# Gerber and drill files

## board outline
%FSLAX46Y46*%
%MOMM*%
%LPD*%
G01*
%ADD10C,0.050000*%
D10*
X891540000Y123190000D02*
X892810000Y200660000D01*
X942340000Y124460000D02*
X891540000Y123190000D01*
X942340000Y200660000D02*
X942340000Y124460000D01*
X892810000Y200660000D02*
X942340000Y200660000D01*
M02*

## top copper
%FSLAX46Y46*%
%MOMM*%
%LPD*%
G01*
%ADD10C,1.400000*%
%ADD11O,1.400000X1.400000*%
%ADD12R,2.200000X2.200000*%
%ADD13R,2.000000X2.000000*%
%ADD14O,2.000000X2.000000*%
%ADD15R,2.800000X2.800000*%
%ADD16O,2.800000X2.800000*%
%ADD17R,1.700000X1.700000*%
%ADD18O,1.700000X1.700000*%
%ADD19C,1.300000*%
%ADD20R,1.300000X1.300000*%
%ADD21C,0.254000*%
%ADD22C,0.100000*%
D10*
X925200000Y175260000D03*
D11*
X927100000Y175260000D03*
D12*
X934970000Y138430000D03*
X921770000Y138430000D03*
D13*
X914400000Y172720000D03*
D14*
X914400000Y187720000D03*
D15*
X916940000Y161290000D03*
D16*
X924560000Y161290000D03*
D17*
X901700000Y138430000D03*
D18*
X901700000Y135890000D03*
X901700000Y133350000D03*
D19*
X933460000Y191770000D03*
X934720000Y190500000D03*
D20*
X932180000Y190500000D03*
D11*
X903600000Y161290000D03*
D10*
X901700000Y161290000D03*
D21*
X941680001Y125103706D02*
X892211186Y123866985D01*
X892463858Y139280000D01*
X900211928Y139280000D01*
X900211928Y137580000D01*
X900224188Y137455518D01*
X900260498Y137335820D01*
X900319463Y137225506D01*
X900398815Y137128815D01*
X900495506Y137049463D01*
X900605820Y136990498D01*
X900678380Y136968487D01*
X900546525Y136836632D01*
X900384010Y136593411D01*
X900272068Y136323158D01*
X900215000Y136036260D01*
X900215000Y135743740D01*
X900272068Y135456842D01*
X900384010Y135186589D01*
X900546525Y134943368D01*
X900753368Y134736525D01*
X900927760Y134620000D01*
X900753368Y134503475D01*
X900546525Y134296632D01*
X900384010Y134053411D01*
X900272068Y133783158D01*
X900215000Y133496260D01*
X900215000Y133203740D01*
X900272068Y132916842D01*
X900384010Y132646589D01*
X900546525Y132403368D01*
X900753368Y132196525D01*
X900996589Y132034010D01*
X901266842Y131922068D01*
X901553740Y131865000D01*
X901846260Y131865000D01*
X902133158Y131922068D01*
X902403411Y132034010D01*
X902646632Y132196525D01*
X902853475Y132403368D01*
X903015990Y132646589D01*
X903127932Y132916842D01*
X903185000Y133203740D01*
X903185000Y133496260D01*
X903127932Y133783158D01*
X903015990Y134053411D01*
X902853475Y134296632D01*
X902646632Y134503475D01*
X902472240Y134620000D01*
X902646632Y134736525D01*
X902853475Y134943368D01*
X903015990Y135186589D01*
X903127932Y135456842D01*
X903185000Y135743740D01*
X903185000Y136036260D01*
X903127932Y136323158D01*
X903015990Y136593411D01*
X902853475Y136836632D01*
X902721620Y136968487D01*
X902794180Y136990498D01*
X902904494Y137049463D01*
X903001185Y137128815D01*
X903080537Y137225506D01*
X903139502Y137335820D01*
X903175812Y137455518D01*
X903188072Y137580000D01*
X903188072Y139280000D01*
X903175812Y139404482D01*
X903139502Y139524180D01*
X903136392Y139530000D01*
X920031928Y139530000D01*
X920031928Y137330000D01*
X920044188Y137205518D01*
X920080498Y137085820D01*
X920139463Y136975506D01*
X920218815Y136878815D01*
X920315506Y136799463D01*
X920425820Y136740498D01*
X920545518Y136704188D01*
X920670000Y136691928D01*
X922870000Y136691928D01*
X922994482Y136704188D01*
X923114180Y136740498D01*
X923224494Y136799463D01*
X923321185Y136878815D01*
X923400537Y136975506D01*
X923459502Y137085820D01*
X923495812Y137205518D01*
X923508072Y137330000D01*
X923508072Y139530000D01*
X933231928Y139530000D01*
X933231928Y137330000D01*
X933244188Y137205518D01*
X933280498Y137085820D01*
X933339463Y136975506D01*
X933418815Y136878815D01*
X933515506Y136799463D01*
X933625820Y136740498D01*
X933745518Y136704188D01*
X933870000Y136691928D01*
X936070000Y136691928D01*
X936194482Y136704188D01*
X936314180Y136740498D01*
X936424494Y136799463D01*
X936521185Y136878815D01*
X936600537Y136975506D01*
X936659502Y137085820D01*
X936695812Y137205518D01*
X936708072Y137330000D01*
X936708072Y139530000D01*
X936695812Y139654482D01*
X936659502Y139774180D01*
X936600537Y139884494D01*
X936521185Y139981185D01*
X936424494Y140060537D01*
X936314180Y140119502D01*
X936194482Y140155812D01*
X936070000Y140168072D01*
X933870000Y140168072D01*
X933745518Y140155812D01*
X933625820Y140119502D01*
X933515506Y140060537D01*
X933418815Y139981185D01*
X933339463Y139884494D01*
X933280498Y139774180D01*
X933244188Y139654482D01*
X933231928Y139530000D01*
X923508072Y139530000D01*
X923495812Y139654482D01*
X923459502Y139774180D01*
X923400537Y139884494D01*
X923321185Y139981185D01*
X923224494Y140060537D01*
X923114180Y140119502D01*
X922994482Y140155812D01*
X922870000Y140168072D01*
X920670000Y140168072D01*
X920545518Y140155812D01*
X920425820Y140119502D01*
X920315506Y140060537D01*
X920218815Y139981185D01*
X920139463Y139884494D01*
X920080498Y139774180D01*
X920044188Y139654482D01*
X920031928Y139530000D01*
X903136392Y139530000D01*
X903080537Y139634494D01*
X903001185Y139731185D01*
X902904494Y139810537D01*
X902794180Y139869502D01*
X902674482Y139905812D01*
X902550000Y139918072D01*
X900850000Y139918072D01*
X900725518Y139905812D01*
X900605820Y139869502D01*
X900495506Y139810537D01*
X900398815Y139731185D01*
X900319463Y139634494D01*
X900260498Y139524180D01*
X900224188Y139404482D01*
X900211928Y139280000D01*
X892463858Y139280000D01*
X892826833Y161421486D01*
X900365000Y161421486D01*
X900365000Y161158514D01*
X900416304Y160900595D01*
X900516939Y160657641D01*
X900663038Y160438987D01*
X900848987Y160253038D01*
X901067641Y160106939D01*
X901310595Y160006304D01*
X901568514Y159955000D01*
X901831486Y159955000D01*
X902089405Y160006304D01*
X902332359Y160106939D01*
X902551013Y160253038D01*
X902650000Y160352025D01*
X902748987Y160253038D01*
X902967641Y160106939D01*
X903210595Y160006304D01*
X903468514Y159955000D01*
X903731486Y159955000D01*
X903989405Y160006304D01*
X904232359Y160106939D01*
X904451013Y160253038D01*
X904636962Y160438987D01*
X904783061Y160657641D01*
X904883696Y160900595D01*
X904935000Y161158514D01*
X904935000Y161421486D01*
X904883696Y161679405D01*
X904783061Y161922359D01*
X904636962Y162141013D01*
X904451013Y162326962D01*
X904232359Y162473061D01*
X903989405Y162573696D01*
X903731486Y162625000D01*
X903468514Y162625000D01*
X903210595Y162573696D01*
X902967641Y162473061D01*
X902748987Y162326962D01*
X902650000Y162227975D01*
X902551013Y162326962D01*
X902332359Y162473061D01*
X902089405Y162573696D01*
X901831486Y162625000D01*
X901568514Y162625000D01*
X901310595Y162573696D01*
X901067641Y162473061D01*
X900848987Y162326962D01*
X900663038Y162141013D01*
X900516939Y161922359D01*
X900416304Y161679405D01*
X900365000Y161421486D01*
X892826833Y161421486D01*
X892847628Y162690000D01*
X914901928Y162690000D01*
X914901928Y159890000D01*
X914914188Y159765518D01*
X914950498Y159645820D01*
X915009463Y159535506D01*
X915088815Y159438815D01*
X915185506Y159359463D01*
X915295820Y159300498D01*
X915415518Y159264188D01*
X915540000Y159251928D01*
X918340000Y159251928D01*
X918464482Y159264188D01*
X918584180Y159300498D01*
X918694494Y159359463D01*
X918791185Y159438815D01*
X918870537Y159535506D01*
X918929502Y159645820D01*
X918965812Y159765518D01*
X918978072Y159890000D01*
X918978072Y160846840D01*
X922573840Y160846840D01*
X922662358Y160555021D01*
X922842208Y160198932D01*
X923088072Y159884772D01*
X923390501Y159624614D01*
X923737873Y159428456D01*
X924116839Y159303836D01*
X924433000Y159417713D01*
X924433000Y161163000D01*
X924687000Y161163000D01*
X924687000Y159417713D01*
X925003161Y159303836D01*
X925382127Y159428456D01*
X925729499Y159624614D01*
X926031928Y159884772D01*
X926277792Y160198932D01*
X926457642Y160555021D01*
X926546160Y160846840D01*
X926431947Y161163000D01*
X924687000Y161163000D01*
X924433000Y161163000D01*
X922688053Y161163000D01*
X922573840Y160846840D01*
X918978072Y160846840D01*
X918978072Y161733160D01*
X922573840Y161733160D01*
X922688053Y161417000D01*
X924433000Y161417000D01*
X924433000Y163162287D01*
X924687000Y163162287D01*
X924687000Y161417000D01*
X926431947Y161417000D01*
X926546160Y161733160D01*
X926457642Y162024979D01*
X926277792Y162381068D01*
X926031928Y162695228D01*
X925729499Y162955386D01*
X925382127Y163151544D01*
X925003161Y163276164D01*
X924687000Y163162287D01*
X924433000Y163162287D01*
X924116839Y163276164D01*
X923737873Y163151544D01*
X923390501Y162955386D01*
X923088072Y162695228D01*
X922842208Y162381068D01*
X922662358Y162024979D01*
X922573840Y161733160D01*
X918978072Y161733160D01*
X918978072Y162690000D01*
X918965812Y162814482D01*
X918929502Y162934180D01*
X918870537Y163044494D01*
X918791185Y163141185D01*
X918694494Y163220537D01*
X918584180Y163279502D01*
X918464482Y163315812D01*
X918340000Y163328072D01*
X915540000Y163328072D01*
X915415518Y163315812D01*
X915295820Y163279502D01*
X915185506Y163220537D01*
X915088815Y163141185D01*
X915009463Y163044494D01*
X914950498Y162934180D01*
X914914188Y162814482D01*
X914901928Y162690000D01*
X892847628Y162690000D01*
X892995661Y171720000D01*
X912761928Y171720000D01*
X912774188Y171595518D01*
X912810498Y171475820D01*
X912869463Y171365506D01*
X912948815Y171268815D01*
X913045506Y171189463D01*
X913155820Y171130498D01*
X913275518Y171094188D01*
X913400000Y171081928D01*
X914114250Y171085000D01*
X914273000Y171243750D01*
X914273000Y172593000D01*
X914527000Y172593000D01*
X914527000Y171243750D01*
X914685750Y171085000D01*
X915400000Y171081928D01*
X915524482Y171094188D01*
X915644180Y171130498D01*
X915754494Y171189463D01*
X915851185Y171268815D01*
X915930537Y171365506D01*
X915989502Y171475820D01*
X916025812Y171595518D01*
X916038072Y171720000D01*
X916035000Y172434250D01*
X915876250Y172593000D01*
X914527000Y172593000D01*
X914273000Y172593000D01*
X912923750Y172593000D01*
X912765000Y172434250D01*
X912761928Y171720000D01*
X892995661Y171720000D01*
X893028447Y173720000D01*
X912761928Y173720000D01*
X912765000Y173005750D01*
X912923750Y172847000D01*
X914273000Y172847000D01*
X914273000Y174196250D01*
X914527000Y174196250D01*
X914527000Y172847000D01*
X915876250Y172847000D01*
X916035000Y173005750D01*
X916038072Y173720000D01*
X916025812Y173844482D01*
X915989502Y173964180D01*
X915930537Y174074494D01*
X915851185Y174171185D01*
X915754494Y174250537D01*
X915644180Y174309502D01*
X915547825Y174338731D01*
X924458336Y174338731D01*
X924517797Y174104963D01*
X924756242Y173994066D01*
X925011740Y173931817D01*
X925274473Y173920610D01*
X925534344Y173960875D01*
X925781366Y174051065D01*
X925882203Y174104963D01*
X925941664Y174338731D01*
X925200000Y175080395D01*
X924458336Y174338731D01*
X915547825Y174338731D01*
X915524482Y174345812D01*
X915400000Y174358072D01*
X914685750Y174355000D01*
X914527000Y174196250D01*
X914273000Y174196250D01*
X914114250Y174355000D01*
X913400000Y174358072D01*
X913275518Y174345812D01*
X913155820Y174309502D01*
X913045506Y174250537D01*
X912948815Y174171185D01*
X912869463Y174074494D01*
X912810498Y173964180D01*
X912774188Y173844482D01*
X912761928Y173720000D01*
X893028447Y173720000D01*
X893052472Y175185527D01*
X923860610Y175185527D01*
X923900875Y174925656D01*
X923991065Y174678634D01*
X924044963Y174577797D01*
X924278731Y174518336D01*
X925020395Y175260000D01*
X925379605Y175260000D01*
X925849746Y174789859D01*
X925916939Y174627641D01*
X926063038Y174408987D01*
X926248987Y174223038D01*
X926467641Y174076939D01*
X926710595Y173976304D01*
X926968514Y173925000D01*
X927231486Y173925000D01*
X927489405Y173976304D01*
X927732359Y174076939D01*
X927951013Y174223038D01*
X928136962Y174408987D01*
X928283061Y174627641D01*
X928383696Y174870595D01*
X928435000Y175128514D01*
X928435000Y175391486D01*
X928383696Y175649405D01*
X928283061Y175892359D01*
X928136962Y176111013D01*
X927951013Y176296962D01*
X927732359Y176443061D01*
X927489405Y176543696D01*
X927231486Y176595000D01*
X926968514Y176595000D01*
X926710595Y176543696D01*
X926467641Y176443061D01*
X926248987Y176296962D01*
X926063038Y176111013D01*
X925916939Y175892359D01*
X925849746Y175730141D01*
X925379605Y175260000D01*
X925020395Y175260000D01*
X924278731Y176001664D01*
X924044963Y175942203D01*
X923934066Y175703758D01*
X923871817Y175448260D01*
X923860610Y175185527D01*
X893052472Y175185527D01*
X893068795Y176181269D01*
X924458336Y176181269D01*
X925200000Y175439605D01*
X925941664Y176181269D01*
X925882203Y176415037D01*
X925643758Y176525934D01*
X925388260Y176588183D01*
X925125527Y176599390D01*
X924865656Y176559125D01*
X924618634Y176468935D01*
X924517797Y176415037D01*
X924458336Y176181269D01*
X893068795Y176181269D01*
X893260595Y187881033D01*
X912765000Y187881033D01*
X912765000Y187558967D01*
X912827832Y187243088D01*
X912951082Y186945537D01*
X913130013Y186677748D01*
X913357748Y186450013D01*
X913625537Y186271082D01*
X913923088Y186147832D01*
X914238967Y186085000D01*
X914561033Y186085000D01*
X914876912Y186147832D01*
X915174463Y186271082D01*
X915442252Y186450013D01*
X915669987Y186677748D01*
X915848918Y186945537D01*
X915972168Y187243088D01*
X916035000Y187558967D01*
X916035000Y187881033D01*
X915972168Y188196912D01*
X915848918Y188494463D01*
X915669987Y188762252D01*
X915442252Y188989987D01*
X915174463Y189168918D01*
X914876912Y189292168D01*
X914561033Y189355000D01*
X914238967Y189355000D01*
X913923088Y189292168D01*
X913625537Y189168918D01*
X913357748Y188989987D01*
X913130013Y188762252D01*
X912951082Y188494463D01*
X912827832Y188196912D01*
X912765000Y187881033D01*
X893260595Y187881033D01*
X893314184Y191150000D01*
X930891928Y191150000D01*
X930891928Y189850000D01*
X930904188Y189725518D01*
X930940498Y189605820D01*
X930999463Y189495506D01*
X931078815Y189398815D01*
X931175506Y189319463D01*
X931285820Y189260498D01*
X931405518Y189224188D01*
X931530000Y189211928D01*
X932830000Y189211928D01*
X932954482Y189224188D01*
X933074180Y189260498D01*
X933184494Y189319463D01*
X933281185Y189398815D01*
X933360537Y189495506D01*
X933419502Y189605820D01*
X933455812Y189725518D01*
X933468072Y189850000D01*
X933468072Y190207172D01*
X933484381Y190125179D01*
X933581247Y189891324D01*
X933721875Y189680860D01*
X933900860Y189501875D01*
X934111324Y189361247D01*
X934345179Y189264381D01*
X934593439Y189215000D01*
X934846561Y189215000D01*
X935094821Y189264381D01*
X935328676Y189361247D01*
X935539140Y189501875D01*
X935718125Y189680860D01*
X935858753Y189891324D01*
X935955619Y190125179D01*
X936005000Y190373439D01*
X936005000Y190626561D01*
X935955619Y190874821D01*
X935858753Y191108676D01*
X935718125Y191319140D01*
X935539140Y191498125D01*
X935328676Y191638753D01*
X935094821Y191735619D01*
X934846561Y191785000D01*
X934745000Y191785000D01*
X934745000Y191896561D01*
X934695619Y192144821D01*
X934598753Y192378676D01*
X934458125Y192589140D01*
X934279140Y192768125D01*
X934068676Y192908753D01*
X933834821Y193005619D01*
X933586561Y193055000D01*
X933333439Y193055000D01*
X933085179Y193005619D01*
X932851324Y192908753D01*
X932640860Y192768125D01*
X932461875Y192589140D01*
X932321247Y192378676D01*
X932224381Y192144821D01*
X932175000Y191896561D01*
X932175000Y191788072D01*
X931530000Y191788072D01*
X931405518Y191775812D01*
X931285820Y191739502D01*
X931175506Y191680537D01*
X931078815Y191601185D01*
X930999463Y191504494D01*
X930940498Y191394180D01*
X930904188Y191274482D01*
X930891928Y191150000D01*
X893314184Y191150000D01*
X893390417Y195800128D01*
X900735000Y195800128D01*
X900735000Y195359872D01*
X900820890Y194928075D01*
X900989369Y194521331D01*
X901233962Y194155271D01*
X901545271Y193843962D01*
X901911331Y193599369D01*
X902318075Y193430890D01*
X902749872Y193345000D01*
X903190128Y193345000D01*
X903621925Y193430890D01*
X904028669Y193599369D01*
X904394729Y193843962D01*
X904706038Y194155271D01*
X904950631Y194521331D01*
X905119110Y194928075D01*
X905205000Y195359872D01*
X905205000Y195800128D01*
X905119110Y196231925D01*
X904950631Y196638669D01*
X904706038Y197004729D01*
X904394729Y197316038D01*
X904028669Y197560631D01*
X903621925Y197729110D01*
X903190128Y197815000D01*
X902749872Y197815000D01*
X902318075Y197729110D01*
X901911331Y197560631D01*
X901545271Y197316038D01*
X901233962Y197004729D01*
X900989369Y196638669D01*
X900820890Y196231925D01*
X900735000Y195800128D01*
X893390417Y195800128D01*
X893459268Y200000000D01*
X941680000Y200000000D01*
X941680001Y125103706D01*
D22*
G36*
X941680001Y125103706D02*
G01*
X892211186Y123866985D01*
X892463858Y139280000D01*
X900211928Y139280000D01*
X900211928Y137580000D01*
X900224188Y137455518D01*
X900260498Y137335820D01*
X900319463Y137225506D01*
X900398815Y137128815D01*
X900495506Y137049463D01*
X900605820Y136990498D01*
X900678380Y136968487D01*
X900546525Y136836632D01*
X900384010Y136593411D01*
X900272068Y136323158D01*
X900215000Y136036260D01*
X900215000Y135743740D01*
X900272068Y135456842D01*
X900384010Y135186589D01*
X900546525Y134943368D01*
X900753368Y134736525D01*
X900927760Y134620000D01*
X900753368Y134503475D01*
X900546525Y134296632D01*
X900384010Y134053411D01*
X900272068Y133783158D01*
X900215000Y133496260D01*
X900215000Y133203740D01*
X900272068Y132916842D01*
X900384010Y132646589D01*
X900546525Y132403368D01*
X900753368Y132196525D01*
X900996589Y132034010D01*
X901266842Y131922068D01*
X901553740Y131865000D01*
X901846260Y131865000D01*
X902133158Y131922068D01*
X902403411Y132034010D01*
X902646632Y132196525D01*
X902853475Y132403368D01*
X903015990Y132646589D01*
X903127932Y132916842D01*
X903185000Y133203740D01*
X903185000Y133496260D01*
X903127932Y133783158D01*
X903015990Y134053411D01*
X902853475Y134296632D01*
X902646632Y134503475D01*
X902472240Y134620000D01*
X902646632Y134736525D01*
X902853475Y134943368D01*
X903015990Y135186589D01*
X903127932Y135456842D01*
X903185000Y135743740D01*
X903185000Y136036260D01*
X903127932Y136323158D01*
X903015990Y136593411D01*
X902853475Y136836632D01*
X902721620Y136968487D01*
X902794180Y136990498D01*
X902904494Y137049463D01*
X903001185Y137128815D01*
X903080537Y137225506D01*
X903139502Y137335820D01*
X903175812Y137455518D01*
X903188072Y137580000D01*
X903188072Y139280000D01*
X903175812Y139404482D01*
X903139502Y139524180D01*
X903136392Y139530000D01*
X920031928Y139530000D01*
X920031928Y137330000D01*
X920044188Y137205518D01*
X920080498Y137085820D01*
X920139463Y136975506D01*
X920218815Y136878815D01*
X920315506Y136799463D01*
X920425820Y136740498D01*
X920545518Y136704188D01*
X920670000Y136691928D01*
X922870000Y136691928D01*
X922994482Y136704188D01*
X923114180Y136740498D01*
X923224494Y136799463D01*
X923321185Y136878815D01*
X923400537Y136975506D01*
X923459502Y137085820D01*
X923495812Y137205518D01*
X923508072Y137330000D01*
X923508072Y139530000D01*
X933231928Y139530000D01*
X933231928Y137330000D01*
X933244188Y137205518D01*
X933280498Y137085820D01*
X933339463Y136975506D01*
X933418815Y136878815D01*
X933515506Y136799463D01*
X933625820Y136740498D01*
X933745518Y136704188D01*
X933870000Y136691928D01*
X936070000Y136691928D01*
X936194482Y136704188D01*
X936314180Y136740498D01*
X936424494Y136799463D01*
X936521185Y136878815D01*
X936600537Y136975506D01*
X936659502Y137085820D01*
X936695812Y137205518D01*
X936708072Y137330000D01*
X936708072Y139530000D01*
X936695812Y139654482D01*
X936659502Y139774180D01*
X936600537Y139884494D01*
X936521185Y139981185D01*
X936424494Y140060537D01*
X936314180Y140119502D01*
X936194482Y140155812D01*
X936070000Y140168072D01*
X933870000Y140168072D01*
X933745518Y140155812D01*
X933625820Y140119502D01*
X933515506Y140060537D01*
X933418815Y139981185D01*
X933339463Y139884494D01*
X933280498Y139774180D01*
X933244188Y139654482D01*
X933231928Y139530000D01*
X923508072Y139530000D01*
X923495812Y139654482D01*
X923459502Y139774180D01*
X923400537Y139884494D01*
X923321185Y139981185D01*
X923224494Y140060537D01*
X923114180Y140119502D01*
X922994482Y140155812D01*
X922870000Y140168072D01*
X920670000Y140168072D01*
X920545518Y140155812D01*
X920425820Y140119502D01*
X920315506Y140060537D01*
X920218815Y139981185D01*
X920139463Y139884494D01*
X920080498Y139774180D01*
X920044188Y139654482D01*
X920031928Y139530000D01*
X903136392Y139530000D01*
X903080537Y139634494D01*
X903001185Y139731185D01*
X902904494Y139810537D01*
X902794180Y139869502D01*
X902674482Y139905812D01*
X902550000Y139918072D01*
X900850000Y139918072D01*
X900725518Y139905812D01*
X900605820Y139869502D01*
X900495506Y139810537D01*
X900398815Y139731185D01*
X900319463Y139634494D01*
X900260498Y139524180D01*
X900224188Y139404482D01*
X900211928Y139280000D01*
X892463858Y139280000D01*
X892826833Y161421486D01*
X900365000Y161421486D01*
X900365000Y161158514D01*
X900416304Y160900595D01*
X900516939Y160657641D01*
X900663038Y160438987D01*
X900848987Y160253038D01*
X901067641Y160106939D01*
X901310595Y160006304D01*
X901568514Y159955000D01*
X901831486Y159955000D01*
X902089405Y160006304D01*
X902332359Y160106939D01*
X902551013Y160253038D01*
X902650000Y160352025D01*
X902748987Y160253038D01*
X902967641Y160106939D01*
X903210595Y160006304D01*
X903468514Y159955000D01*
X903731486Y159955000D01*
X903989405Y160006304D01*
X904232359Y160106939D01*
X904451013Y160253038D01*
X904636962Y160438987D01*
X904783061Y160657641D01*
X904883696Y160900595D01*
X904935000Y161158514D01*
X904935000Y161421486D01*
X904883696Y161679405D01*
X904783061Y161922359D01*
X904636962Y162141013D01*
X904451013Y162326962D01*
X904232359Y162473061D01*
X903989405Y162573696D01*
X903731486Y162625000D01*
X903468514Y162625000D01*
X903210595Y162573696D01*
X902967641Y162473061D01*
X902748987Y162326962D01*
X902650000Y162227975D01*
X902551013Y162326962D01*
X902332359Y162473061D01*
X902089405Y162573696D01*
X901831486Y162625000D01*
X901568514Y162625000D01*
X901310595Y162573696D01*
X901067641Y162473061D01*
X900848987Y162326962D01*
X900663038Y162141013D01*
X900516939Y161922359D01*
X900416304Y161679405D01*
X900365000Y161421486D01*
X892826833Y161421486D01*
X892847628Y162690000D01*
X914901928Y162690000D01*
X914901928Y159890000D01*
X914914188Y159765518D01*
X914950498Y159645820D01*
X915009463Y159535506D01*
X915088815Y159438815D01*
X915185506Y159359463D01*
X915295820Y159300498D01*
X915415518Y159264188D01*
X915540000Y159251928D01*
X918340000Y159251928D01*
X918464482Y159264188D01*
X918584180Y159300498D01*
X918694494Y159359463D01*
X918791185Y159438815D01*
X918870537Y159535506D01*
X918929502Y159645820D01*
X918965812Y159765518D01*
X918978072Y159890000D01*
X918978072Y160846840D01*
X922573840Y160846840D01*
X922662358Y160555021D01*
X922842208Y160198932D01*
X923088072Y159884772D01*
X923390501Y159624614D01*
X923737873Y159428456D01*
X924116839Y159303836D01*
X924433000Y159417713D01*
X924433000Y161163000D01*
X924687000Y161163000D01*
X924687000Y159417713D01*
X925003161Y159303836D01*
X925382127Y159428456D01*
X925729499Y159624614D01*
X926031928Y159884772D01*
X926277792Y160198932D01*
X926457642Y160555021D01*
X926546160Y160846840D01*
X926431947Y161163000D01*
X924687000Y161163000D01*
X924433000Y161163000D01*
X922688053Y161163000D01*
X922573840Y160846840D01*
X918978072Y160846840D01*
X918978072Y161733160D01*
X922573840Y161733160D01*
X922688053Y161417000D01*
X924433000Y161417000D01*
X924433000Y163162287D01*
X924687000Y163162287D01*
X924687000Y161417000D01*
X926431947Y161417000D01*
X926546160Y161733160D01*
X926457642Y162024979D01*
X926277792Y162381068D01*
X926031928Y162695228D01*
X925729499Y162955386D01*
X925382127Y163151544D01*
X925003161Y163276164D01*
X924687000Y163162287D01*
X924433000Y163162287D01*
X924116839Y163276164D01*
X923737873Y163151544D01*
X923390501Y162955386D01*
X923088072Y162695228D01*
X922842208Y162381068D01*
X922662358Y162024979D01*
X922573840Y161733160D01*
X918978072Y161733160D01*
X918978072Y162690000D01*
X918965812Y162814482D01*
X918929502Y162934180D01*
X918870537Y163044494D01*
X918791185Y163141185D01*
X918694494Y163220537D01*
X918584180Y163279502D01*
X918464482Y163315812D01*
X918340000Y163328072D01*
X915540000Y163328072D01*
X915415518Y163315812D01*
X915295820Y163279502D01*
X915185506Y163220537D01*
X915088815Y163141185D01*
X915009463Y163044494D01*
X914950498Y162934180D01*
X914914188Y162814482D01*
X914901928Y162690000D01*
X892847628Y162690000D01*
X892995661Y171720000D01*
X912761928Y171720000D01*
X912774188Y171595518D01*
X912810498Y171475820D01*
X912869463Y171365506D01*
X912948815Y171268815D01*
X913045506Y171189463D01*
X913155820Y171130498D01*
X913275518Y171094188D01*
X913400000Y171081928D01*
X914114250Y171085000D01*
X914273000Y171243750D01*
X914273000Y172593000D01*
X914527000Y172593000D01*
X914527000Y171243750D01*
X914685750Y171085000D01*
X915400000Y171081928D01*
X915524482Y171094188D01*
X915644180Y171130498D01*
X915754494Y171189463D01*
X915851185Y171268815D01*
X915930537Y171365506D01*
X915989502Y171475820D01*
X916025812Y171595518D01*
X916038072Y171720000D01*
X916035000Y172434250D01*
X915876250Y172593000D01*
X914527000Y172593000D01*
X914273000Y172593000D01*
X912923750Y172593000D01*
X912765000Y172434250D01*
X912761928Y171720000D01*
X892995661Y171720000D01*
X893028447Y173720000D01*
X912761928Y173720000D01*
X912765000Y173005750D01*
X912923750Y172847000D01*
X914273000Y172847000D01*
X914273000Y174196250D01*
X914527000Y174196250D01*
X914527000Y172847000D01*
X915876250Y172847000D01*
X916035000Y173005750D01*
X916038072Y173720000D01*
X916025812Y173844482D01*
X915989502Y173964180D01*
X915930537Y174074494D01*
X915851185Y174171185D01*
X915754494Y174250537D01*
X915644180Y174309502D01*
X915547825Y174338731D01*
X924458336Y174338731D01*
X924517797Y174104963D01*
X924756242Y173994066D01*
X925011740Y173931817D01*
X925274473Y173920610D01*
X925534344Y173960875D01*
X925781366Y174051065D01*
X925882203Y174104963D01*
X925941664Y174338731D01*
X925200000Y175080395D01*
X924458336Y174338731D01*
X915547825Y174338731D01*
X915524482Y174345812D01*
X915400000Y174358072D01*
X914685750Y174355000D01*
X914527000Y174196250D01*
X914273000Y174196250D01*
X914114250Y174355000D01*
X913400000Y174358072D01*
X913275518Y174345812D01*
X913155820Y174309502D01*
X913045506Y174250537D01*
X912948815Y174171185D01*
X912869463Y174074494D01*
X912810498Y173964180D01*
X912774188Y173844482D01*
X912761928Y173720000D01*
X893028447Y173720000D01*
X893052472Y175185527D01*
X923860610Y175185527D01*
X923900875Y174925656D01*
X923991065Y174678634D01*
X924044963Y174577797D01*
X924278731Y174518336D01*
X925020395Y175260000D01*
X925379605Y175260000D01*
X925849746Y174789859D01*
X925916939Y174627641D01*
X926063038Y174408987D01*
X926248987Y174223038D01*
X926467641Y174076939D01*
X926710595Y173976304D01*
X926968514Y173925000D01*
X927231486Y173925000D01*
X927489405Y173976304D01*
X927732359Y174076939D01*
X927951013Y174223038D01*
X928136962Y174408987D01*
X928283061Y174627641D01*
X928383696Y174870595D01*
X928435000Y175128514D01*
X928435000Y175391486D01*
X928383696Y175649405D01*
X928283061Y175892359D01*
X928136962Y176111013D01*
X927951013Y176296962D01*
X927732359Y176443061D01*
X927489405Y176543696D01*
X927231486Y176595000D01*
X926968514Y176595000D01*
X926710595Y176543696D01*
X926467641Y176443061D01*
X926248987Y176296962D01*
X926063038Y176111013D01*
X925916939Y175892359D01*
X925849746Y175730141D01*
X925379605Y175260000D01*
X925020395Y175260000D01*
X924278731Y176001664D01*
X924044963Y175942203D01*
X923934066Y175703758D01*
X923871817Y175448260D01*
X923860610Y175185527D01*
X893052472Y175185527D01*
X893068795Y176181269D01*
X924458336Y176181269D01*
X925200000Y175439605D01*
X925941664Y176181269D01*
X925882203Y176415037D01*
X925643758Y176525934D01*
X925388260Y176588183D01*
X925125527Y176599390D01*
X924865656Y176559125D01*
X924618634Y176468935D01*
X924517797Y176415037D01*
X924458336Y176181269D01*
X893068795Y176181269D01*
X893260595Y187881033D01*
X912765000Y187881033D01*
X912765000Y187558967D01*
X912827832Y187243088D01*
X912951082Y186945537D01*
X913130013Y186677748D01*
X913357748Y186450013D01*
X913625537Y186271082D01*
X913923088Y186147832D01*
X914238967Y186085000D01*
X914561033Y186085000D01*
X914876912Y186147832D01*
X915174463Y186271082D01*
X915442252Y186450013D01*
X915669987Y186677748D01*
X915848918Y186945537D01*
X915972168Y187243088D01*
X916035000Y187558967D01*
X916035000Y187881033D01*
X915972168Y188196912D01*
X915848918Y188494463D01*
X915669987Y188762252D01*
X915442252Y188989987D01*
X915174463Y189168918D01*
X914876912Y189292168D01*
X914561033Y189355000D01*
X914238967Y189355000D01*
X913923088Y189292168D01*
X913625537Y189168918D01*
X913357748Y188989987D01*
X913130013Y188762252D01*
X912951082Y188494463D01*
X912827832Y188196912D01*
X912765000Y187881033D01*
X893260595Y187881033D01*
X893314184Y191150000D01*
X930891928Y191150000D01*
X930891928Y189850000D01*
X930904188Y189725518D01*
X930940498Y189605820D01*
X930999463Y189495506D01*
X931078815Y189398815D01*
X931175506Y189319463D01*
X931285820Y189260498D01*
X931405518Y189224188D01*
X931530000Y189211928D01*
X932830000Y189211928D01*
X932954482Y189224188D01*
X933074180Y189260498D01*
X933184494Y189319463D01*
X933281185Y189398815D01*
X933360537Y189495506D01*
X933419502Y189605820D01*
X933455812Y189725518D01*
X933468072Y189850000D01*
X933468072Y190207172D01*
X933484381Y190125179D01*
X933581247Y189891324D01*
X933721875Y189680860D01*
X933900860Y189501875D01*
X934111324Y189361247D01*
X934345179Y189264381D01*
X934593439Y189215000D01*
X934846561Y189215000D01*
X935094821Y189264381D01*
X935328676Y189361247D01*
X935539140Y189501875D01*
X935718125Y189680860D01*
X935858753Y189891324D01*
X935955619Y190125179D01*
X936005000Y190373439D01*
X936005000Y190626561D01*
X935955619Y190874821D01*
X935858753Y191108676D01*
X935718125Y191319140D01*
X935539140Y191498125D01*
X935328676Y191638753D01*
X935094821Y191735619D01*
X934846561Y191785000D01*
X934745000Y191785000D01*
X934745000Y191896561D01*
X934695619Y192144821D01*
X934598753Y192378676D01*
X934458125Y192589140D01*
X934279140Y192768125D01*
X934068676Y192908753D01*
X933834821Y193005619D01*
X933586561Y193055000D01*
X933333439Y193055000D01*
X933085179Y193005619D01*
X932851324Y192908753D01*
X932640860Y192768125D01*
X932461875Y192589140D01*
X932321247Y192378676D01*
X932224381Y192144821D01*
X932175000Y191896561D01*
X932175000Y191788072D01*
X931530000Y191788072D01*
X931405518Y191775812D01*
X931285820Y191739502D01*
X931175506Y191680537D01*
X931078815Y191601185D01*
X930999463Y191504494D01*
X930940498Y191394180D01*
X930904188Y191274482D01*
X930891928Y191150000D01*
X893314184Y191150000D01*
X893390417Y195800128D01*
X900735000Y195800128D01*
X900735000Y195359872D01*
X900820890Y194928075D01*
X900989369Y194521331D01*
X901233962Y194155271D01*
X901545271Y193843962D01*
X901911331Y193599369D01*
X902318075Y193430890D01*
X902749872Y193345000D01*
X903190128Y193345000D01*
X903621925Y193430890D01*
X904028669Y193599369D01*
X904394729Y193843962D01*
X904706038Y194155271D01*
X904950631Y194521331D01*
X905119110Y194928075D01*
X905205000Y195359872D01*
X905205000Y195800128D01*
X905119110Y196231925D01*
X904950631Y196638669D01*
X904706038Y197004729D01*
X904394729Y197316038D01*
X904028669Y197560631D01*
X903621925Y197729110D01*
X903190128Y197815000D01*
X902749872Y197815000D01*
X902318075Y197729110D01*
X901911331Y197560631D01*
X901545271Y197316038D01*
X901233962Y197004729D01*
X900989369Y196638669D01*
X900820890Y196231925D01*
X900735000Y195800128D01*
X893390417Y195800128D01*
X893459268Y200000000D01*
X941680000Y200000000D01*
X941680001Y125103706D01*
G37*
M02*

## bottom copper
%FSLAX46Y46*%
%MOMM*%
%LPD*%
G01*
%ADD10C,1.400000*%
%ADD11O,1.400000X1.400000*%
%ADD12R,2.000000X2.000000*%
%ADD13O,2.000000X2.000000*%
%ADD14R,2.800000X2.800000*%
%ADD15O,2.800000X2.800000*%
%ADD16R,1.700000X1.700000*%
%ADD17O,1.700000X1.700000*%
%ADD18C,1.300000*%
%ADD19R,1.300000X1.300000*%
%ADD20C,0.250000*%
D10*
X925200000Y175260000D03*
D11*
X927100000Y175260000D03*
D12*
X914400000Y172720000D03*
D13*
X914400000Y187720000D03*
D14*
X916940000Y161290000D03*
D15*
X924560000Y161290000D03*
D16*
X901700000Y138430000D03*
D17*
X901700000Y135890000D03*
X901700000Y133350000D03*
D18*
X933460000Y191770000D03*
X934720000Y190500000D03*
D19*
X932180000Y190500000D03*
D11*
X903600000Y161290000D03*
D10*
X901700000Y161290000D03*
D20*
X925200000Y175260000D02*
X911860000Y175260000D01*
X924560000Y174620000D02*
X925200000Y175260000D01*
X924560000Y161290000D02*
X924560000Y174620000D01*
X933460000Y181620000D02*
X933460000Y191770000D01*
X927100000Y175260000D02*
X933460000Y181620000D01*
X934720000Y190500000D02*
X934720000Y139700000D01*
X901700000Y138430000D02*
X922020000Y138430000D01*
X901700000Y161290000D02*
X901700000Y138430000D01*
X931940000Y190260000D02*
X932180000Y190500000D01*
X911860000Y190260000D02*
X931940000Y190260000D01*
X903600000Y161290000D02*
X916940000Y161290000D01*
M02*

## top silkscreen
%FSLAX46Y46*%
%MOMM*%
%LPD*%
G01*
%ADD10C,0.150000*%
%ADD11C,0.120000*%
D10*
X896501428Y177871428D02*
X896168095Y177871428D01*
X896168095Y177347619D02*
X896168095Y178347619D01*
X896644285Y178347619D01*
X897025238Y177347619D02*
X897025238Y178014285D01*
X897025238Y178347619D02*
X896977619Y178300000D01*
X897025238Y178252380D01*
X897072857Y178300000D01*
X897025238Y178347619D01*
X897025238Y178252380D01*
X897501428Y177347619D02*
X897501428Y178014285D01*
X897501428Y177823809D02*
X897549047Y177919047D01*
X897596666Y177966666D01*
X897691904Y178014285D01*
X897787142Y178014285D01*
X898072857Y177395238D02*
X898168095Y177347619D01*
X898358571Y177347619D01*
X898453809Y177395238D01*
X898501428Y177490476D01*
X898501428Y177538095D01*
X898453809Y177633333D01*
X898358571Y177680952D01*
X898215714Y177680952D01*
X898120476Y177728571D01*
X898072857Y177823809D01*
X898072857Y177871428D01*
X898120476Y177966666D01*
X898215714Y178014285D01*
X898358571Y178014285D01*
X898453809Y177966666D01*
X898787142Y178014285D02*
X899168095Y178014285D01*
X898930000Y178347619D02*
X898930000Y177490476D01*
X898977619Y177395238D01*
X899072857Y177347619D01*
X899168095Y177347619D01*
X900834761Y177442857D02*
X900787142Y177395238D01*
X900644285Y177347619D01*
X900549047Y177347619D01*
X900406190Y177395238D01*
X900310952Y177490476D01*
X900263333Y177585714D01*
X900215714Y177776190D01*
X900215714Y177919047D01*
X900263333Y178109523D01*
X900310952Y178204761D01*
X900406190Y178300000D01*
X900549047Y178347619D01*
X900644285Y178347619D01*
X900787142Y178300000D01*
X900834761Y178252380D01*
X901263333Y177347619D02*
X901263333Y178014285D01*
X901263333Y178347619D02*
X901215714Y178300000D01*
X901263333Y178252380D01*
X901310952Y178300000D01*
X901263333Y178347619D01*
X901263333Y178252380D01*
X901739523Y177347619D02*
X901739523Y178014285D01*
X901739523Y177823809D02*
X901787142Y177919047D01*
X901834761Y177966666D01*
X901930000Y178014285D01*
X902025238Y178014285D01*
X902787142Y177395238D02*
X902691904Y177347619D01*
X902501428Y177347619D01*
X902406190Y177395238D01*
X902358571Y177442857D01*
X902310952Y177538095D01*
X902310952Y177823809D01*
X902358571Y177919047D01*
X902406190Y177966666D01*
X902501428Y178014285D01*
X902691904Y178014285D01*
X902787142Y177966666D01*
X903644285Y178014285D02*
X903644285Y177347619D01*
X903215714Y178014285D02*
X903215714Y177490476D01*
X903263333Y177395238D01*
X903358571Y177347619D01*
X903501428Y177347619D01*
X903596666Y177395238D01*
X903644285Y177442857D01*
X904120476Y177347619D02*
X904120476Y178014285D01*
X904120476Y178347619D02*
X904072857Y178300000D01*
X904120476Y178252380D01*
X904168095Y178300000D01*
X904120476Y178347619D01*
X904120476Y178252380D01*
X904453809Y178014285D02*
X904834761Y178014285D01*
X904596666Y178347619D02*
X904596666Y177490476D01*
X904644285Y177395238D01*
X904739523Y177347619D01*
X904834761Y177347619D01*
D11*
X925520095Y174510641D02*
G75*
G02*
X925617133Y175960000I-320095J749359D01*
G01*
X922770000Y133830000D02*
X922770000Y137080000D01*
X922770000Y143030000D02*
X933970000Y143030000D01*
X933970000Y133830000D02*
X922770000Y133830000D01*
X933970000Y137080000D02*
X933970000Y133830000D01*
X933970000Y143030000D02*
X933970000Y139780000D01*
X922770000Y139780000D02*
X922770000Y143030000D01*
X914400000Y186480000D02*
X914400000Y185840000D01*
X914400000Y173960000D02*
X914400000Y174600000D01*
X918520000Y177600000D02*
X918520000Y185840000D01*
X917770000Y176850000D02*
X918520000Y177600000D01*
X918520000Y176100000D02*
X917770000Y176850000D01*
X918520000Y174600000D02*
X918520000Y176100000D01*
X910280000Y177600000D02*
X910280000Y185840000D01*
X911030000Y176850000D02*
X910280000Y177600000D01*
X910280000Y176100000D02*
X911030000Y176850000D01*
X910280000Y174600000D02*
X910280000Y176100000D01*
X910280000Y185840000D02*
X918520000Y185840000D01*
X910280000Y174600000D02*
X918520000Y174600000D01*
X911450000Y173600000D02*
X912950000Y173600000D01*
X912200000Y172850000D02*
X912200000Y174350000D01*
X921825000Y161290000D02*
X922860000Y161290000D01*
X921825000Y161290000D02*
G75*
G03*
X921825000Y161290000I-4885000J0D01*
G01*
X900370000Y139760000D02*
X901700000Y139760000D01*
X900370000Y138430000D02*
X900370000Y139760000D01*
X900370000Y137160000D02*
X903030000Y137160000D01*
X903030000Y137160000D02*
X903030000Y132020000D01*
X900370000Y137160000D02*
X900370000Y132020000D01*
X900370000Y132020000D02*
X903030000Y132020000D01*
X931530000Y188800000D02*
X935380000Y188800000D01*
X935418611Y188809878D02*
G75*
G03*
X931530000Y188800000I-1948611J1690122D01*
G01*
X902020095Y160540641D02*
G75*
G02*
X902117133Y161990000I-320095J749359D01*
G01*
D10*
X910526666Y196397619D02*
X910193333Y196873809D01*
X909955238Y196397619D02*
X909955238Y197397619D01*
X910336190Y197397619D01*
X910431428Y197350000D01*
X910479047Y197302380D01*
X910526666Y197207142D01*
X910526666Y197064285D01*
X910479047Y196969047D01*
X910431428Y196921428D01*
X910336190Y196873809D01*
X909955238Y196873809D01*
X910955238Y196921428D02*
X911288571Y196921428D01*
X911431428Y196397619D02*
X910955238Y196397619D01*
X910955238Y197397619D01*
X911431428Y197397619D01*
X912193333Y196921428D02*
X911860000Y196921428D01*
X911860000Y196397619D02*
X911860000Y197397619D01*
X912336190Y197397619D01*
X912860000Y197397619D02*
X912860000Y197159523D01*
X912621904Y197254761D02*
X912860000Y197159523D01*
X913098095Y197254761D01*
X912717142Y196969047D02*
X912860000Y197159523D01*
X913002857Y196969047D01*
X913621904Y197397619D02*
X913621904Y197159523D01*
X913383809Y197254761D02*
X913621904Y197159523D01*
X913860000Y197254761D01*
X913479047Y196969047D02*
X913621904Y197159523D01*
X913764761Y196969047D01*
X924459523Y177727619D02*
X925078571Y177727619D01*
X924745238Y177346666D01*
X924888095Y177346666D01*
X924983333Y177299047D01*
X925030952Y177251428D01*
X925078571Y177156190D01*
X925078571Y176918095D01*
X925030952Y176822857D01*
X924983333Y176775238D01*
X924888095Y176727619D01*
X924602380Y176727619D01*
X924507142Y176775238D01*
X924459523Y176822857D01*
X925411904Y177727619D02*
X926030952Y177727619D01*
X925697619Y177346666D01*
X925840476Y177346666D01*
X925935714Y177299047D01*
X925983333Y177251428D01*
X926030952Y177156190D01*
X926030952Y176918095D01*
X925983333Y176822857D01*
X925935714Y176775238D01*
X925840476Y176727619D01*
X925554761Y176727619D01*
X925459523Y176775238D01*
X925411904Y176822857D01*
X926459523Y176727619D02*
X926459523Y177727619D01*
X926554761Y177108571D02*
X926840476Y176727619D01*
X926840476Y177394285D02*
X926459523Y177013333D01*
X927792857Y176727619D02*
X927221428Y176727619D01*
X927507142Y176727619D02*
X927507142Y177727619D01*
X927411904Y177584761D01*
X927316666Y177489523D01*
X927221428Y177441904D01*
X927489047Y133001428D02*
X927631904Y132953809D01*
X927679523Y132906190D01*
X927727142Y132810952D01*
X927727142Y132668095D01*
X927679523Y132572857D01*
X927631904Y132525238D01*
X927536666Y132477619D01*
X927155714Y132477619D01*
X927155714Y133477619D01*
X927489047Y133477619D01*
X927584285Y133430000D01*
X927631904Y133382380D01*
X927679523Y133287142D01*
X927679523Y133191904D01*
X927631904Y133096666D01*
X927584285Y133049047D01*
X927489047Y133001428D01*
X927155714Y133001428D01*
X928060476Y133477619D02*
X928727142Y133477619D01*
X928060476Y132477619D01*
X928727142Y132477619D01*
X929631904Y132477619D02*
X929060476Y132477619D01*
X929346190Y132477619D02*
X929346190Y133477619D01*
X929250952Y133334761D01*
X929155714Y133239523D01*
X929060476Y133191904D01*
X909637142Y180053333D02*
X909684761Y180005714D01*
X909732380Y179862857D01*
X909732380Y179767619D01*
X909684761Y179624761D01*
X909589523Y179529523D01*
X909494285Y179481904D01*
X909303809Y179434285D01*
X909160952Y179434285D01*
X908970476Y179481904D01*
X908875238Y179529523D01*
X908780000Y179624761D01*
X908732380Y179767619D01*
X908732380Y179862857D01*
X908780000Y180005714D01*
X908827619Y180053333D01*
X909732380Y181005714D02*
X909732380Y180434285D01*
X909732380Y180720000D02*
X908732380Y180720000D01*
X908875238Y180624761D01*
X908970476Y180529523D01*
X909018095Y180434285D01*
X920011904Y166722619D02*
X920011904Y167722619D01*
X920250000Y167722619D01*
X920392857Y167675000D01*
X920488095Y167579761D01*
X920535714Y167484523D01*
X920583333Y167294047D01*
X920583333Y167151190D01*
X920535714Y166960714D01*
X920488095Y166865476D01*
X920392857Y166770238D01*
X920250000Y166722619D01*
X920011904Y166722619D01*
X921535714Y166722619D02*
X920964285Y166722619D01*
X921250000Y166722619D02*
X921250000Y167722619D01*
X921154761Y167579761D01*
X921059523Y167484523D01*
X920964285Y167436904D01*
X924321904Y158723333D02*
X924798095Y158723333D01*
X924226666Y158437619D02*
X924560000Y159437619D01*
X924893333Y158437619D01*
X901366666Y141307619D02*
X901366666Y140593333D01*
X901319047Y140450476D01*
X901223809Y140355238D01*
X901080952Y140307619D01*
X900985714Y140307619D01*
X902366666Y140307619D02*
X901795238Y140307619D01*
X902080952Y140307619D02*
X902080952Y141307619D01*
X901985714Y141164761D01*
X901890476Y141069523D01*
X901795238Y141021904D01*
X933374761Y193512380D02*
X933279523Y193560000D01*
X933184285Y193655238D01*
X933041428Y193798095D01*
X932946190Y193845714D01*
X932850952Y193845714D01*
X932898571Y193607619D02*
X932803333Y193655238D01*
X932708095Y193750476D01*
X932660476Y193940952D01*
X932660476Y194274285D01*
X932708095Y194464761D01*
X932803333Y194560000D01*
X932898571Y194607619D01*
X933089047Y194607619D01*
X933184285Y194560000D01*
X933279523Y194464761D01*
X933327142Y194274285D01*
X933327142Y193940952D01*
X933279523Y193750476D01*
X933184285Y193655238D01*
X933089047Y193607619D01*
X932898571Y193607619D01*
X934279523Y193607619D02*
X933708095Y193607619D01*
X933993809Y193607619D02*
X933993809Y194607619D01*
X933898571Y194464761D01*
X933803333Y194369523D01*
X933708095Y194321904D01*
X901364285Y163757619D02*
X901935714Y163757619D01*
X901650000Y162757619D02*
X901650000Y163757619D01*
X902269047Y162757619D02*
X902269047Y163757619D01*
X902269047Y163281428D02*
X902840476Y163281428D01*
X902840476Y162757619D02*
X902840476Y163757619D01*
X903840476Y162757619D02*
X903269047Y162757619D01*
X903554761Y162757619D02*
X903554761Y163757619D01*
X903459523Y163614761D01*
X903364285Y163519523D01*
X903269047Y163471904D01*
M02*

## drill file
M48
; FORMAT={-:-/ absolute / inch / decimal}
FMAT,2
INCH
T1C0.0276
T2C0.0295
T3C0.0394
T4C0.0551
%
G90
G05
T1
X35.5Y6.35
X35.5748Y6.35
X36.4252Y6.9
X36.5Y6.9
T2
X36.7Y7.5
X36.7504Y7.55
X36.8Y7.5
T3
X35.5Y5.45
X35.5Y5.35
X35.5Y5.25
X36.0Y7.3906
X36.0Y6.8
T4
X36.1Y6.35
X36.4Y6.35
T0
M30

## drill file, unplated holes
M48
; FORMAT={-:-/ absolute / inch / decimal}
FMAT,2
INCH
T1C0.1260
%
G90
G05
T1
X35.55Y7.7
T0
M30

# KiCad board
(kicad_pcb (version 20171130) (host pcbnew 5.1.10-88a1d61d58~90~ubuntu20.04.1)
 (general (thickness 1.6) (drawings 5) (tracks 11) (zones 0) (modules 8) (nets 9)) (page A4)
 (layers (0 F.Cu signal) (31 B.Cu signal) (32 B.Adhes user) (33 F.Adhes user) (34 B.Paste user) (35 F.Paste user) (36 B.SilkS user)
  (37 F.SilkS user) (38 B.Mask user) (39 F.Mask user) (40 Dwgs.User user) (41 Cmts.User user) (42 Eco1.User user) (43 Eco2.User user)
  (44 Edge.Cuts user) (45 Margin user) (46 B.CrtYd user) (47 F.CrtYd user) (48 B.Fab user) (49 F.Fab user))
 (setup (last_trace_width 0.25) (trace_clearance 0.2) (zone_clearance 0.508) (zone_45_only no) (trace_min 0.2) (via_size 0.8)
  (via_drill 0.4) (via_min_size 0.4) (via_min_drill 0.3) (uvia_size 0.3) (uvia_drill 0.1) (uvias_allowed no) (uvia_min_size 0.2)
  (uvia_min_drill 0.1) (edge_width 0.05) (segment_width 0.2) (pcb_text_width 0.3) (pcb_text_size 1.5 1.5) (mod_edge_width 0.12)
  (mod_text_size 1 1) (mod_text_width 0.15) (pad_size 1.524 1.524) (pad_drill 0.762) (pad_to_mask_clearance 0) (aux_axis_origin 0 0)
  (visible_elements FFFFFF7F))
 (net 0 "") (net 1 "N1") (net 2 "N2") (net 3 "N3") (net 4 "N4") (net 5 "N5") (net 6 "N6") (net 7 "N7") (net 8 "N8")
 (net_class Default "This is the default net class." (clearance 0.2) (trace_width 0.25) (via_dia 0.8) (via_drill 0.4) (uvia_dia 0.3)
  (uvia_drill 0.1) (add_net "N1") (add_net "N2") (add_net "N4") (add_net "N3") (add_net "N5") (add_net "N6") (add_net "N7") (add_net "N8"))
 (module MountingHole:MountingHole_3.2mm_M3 (layer F.Cu) (at 902.97 -195.58)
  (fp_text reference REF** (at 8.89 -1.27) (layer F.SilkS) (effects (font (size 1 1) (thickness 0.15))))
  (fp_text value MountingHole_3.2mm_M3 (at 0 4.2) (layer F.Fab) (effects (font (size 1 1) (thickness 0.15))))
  (pad 1 np_thru_hole circle (at 0 0) (size 3.2 3.2) (drill 3.2) (layers *.Cu *.Mask)))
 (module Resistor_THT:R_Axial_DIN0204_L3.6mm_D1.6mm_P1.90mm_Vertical (layer F.Cu) (at 925.2 -175.26)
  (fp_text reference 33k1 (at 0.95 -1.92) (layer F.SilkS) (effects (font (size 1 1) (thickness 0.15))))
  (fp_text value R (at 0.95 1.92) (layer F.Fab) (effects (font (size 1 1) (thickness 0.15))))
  (fp_arc (start 0 0) (end 0.417133 -0.7) (angle -233.92106) (layer F.SilkS) (width 0.12))
  (pad 1 thru_hole circle (at 0 0) (size 1.4 1.4) (drill 0.7) (layers *.Cu *.Mask) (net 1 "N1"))
  (pad 2 thru_hole oval (at 1.9 0) (size 1.4 1.4) (drill 0.7) (layers *.Cu *.Mask) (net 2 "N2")))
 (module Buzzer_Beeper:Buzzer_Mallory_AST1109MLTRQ (layer F.Cu) (at 928.37 -138.43)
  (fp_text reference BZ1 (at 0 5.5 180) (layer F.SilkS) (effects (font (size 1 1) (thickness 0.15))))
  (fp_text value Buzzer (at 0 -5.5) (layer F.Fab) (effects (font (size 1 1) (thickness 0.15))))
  (fp_line (start -5.6 4.6) (end -5.6 1.35) (layer F.SilkS) (width 0.12))
  (fp_line (start -5.6 -4.6) (end 5.6 -4.6) (layer F.SilkS) (width 0.12))
  (fp_line (start 5.6 4.6) (end -5.6 4.6) (layer F.SilkS) (width 0.12))
  (fp_line (start 5.6 1.35) (end 5.6 4.6) (layer F.SilkS) (width 0.12))
  (fp_line (start 5.6 -4.6) (end 5.6 -1.35) (layer F.SilkS) (width 0.12))
  (fp_line (start -5.6 -1.35) (end -5.6 -4.6) (layer F.SilkS) (width 0.12))
  (pad 2 smd rect (at 6.6 0) (size 2.2 2.2) (layers F.Cu F.Paste F.Mask) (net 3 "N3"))
  (pad 1 smd rect (at -6.6 0) (size 2.2 2.2) (layers F.Cu F.Paste F.Mask) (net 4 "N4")))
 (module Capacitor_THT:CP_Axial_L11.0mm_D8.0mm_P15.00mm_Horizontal (layer F.Cu) (at 914.4 -172.72 90)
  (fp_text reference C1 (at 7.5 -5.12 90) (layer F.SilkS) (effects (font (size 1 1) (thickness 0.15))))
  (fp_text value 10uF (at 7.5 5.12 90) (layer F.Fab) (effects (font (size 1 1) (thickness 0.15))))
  (fp_line (start 13.76 0) (end 13.12 0) (layer F.SilkS) (width 0.12))
  (fp_line (start 1.24 0) (end 1.88 0) (layer F.SilkS) (width 0.12))
  (fp_line (start 4.88 4.12) (end 13.12 4.12) (layer F.SilkS) (width 0.12))
  (fp_line (start 4.13 3.37) (end 4.88 4.12) (layer F.SilkS) (width 0.12))
  (fp_line (start 3.38 4.12) (end 4.13 3.37) (layer F.SilkS) (width 0.12))
  (fp_line (start 1.88 4.12) (end 3.38 4.12) (layer F.SilkS) (width 0.12))
  (fp_line (start 4.88 -4.12) (end 13.12 -4.12) (layer F.SilkS) (width 0.12))
  (fp_line (start 4.13 -3.37) (end 4.88 -4.12) (layer F.SilkS) (width 0.12))
  (fp_line (start 3.38 -4.12) (end 4.13 -3.37) (layer F.SilkS) (width 0.12))
  (fp_line (start 1.88 -4.12) (end 3.38 -4.12) (layer F.SilkS) (width 0.12))
  (fp_line (start 13.12 -4.12) (end 13.12 4.12) (layer F.SilkS) (width 0.12))
  (fp_line (start 1.88 -4.12) (end 1.88 4.12) (layer F.SilkS) (width 0.12))
  (fp_line (start 0.88 -2.95) (end 0.88 -1.45) (layer F.SilkS) (width 0.12))
  (fp_line (start 0.13 -2.2) (end 1.63 -2.2) (layer F.SilkS) (width 0.12))
  (pad 1 thru_hole rect (at 0 0 90) (size 2 2) (drill 1) (layers *.Cu *.Mask) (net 1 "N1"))
  (pad 2 thru_hole oval (at 15 0 90) (size 2 2) (drill 1) (layers *.Cu *.Mask) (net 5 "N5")))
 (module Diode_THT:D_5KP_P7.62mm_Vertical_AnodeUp (layer F.Cu) (at 916.94 -161.29)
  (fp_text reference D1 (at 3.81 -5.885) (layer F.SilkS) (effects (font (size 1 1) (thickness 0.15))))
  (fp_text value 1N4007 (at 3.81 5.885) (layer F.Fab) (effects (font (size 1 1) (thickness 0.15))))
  (fp_line (start 4.885 0) (end 5.92 0) (layer F.SilkS) (width 0.12))
  (fp_circle (center 0 0) (end 4.885 0) (layer F.SilkS) (width 0.12))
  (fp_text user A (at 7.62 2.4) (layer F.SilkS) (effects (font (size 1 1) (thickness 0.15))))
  (pad 1 thru_hole rect (at 0 0) (size 2.8 2.8) (drill 1.4) (layers *.Cu *.Mask) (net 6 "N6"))
  (pad 2 thru_hole oval (at 7.62 0) (size 2.8 2.8) (drill 1.4) (layers *.Cu *.Mask) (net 1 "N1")))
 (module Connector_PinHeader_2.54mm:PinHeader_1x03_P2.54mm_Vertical (layer F.Cu) (at 901.7 -138.43)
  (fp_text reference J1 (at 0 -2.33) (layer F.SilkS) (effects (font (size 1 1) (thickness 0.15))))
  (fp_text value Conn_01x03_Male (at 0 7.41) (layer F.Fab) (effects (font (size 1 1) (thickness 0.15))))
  (fp_line (start -1.33 -1.33) (end 0 -1.33) (layer F.SilkS) (width 0.12))
  (fp_line (start -1.33 0) (end -1.33 -1.33) (layer F.SilkS) (width 0.12))
  (fp_line (start -1.33 1.27) (end 1.33 1.27) (layer F.SilkS) (width 0.12))
  (fp_line (start 1.33 1.27) (end 1.33 6.41) (layer F.SilkS) (width 0.12))
  (fp_line (start -1.33 1.27) (end -1.33 6.41) (layer F.SilkS) (width 0.12))
  (fp_line (start -1.33 6.41) (end 1.33 6.41) (layer F.SilkS) (width 0.12))
  (pad 1 thru_hole rect (at 0 0) (size 1.7 1.7) (drill 1) (layers *.Cu *.Mask) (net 4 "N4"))
  (pad 2 thru_hole oval (at 0 2.54) (size 1.7 1.7) (drill 1) (layers *.Cu *.Mask) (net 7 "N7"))
  (pad 3 thru_hole oval (at 0 5.08) (size 1.7 1.7) (drill 1) (layers *.Cu *.Mask) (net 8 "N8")))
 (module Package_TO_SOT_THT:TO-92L (layer F.Cu) (at 932.18 -190.5)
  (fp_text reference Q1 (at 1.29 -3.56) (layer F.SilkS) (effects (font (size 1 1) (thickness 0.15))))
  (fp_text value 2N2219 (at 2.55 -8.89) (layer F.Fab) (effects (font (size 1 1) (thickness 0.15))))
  (fp_line (start -0.65 1.7) (end 3.2 1.7) (layer F.SilkS) (width 0.12))
  (fp_arc (start 1.29 0) (end -0.65 1.7) (angle 262.164354) (layer F.SilkS) (width 0.12))
  (pad 2 thru_hole circle (at 1.28 -1.27) (size 1.3 1.3) (drill 0.75) (layers *.Cu *.Mask) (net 2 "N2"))
  (pad 3 thru_hole circle (at 2.54 0) (size 1.3 1.3) (drill 0.75) (layers *.Cu *.Mask) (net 3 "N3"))
  (pad 1 thru_hole rect (at 0 0) (size 1.3 1.3) (drill 0.75) (layers *.Cu *.Mask) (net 5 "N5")))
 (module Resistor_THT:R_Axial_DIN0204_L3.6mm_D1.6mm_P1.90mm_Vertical (layer F.Cu) (at 901.7 -161.29)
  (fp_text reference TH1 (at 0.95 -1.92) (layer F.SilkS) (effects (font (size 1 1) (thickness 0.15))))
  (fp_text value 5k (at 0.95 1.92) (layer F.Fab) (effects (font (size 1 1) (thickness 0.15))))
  (fp_arc (start 0 0) (end 0.417133 -0.7) (angle -233.92106) (layer F.SilkS) (width 0.12))
  (pad 2 thru_hole oval (at 1.9 0) (size 1.4 1.4) (drill 0.7) (layers *.Cu *.Mask) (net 6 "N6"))
  (pad 1 thru_hole circle (at 0 0) (size 1.4 1.4) (drill 0.7) (layers *.Cu *.Mask) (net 4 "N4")))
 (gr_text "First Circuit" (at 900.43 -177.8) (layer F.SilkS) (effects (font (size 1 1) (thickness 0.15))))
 (gr_line (start 891.54 -123.19) (end 892.81 -200.66) (layer Edge.Cuts) (width 0.05))
 (gr_line (start 942.34 -124.46) (end 891.54 -123.19) (layer Edge.Cuts) (width 0.05))
 (gr_line (start 942.34 -200.66) (end 942.34 -124.46) (layer Edge.Cuts) (width 0.05))
 (gr_line (start 892.81 -200.66) (end 942.34 -200.66) (layer Edge.Cuts) (width 0.05))
 (segment (start 925.2 -175.26) (end 911.86 -175.26) (width 0.25) (layer B.Cu) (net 1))
 (segment (start 924.56 -174.62) (end 925.2 -175.26) (width 0.25) (layer B.Cu) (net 1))
 (segment (start 924.56 -161.29) (end 924.56 -174.62) (width 0.25) (layer B.Cu) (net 1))
 (segment (start 933.46 -181.62) (end 933.46 -191.77) (width 0.25) (layer B.Cu) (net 2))
 (segment (start 927.1 -175.26) (end 933.46 -181.62) (width 0.25) (layer B.Cu) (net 2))
 (segment (start 934.72 -190.5) (end 934.72 -139.7) (width 0.25) (layer B.Cu) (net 3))
 (segment (start 901.7 -138.43) (end 922.02 -138.43) (width 0.25) (layer B.Cu) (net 4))
 (segment (start 901.7 -161.29) (end 901.7 -138.43) (width 0.25) (layer B.Cu) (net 4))
 (segment (start 931.94 -190.26) (end 932.18 -190.5) (width 0.25) (layer B.Cu) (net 5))
 (segment (start 911.86 -190.26) (end 931.94 -190.26) (width 0.25) (layer B.Cu) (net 5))
 (segment (start 903.6 -161.29) (end 916.94 -161.29) (width 0.25) (layer B.Cu) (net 6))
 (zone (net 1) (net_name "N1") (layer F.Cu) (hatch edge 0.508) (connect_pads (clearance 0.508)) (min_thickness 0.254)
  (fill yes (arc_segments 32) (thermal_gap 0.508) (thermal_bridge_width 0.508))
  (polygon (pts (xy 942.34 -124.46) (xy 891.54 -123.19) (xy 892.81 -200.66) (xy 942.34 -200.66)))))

